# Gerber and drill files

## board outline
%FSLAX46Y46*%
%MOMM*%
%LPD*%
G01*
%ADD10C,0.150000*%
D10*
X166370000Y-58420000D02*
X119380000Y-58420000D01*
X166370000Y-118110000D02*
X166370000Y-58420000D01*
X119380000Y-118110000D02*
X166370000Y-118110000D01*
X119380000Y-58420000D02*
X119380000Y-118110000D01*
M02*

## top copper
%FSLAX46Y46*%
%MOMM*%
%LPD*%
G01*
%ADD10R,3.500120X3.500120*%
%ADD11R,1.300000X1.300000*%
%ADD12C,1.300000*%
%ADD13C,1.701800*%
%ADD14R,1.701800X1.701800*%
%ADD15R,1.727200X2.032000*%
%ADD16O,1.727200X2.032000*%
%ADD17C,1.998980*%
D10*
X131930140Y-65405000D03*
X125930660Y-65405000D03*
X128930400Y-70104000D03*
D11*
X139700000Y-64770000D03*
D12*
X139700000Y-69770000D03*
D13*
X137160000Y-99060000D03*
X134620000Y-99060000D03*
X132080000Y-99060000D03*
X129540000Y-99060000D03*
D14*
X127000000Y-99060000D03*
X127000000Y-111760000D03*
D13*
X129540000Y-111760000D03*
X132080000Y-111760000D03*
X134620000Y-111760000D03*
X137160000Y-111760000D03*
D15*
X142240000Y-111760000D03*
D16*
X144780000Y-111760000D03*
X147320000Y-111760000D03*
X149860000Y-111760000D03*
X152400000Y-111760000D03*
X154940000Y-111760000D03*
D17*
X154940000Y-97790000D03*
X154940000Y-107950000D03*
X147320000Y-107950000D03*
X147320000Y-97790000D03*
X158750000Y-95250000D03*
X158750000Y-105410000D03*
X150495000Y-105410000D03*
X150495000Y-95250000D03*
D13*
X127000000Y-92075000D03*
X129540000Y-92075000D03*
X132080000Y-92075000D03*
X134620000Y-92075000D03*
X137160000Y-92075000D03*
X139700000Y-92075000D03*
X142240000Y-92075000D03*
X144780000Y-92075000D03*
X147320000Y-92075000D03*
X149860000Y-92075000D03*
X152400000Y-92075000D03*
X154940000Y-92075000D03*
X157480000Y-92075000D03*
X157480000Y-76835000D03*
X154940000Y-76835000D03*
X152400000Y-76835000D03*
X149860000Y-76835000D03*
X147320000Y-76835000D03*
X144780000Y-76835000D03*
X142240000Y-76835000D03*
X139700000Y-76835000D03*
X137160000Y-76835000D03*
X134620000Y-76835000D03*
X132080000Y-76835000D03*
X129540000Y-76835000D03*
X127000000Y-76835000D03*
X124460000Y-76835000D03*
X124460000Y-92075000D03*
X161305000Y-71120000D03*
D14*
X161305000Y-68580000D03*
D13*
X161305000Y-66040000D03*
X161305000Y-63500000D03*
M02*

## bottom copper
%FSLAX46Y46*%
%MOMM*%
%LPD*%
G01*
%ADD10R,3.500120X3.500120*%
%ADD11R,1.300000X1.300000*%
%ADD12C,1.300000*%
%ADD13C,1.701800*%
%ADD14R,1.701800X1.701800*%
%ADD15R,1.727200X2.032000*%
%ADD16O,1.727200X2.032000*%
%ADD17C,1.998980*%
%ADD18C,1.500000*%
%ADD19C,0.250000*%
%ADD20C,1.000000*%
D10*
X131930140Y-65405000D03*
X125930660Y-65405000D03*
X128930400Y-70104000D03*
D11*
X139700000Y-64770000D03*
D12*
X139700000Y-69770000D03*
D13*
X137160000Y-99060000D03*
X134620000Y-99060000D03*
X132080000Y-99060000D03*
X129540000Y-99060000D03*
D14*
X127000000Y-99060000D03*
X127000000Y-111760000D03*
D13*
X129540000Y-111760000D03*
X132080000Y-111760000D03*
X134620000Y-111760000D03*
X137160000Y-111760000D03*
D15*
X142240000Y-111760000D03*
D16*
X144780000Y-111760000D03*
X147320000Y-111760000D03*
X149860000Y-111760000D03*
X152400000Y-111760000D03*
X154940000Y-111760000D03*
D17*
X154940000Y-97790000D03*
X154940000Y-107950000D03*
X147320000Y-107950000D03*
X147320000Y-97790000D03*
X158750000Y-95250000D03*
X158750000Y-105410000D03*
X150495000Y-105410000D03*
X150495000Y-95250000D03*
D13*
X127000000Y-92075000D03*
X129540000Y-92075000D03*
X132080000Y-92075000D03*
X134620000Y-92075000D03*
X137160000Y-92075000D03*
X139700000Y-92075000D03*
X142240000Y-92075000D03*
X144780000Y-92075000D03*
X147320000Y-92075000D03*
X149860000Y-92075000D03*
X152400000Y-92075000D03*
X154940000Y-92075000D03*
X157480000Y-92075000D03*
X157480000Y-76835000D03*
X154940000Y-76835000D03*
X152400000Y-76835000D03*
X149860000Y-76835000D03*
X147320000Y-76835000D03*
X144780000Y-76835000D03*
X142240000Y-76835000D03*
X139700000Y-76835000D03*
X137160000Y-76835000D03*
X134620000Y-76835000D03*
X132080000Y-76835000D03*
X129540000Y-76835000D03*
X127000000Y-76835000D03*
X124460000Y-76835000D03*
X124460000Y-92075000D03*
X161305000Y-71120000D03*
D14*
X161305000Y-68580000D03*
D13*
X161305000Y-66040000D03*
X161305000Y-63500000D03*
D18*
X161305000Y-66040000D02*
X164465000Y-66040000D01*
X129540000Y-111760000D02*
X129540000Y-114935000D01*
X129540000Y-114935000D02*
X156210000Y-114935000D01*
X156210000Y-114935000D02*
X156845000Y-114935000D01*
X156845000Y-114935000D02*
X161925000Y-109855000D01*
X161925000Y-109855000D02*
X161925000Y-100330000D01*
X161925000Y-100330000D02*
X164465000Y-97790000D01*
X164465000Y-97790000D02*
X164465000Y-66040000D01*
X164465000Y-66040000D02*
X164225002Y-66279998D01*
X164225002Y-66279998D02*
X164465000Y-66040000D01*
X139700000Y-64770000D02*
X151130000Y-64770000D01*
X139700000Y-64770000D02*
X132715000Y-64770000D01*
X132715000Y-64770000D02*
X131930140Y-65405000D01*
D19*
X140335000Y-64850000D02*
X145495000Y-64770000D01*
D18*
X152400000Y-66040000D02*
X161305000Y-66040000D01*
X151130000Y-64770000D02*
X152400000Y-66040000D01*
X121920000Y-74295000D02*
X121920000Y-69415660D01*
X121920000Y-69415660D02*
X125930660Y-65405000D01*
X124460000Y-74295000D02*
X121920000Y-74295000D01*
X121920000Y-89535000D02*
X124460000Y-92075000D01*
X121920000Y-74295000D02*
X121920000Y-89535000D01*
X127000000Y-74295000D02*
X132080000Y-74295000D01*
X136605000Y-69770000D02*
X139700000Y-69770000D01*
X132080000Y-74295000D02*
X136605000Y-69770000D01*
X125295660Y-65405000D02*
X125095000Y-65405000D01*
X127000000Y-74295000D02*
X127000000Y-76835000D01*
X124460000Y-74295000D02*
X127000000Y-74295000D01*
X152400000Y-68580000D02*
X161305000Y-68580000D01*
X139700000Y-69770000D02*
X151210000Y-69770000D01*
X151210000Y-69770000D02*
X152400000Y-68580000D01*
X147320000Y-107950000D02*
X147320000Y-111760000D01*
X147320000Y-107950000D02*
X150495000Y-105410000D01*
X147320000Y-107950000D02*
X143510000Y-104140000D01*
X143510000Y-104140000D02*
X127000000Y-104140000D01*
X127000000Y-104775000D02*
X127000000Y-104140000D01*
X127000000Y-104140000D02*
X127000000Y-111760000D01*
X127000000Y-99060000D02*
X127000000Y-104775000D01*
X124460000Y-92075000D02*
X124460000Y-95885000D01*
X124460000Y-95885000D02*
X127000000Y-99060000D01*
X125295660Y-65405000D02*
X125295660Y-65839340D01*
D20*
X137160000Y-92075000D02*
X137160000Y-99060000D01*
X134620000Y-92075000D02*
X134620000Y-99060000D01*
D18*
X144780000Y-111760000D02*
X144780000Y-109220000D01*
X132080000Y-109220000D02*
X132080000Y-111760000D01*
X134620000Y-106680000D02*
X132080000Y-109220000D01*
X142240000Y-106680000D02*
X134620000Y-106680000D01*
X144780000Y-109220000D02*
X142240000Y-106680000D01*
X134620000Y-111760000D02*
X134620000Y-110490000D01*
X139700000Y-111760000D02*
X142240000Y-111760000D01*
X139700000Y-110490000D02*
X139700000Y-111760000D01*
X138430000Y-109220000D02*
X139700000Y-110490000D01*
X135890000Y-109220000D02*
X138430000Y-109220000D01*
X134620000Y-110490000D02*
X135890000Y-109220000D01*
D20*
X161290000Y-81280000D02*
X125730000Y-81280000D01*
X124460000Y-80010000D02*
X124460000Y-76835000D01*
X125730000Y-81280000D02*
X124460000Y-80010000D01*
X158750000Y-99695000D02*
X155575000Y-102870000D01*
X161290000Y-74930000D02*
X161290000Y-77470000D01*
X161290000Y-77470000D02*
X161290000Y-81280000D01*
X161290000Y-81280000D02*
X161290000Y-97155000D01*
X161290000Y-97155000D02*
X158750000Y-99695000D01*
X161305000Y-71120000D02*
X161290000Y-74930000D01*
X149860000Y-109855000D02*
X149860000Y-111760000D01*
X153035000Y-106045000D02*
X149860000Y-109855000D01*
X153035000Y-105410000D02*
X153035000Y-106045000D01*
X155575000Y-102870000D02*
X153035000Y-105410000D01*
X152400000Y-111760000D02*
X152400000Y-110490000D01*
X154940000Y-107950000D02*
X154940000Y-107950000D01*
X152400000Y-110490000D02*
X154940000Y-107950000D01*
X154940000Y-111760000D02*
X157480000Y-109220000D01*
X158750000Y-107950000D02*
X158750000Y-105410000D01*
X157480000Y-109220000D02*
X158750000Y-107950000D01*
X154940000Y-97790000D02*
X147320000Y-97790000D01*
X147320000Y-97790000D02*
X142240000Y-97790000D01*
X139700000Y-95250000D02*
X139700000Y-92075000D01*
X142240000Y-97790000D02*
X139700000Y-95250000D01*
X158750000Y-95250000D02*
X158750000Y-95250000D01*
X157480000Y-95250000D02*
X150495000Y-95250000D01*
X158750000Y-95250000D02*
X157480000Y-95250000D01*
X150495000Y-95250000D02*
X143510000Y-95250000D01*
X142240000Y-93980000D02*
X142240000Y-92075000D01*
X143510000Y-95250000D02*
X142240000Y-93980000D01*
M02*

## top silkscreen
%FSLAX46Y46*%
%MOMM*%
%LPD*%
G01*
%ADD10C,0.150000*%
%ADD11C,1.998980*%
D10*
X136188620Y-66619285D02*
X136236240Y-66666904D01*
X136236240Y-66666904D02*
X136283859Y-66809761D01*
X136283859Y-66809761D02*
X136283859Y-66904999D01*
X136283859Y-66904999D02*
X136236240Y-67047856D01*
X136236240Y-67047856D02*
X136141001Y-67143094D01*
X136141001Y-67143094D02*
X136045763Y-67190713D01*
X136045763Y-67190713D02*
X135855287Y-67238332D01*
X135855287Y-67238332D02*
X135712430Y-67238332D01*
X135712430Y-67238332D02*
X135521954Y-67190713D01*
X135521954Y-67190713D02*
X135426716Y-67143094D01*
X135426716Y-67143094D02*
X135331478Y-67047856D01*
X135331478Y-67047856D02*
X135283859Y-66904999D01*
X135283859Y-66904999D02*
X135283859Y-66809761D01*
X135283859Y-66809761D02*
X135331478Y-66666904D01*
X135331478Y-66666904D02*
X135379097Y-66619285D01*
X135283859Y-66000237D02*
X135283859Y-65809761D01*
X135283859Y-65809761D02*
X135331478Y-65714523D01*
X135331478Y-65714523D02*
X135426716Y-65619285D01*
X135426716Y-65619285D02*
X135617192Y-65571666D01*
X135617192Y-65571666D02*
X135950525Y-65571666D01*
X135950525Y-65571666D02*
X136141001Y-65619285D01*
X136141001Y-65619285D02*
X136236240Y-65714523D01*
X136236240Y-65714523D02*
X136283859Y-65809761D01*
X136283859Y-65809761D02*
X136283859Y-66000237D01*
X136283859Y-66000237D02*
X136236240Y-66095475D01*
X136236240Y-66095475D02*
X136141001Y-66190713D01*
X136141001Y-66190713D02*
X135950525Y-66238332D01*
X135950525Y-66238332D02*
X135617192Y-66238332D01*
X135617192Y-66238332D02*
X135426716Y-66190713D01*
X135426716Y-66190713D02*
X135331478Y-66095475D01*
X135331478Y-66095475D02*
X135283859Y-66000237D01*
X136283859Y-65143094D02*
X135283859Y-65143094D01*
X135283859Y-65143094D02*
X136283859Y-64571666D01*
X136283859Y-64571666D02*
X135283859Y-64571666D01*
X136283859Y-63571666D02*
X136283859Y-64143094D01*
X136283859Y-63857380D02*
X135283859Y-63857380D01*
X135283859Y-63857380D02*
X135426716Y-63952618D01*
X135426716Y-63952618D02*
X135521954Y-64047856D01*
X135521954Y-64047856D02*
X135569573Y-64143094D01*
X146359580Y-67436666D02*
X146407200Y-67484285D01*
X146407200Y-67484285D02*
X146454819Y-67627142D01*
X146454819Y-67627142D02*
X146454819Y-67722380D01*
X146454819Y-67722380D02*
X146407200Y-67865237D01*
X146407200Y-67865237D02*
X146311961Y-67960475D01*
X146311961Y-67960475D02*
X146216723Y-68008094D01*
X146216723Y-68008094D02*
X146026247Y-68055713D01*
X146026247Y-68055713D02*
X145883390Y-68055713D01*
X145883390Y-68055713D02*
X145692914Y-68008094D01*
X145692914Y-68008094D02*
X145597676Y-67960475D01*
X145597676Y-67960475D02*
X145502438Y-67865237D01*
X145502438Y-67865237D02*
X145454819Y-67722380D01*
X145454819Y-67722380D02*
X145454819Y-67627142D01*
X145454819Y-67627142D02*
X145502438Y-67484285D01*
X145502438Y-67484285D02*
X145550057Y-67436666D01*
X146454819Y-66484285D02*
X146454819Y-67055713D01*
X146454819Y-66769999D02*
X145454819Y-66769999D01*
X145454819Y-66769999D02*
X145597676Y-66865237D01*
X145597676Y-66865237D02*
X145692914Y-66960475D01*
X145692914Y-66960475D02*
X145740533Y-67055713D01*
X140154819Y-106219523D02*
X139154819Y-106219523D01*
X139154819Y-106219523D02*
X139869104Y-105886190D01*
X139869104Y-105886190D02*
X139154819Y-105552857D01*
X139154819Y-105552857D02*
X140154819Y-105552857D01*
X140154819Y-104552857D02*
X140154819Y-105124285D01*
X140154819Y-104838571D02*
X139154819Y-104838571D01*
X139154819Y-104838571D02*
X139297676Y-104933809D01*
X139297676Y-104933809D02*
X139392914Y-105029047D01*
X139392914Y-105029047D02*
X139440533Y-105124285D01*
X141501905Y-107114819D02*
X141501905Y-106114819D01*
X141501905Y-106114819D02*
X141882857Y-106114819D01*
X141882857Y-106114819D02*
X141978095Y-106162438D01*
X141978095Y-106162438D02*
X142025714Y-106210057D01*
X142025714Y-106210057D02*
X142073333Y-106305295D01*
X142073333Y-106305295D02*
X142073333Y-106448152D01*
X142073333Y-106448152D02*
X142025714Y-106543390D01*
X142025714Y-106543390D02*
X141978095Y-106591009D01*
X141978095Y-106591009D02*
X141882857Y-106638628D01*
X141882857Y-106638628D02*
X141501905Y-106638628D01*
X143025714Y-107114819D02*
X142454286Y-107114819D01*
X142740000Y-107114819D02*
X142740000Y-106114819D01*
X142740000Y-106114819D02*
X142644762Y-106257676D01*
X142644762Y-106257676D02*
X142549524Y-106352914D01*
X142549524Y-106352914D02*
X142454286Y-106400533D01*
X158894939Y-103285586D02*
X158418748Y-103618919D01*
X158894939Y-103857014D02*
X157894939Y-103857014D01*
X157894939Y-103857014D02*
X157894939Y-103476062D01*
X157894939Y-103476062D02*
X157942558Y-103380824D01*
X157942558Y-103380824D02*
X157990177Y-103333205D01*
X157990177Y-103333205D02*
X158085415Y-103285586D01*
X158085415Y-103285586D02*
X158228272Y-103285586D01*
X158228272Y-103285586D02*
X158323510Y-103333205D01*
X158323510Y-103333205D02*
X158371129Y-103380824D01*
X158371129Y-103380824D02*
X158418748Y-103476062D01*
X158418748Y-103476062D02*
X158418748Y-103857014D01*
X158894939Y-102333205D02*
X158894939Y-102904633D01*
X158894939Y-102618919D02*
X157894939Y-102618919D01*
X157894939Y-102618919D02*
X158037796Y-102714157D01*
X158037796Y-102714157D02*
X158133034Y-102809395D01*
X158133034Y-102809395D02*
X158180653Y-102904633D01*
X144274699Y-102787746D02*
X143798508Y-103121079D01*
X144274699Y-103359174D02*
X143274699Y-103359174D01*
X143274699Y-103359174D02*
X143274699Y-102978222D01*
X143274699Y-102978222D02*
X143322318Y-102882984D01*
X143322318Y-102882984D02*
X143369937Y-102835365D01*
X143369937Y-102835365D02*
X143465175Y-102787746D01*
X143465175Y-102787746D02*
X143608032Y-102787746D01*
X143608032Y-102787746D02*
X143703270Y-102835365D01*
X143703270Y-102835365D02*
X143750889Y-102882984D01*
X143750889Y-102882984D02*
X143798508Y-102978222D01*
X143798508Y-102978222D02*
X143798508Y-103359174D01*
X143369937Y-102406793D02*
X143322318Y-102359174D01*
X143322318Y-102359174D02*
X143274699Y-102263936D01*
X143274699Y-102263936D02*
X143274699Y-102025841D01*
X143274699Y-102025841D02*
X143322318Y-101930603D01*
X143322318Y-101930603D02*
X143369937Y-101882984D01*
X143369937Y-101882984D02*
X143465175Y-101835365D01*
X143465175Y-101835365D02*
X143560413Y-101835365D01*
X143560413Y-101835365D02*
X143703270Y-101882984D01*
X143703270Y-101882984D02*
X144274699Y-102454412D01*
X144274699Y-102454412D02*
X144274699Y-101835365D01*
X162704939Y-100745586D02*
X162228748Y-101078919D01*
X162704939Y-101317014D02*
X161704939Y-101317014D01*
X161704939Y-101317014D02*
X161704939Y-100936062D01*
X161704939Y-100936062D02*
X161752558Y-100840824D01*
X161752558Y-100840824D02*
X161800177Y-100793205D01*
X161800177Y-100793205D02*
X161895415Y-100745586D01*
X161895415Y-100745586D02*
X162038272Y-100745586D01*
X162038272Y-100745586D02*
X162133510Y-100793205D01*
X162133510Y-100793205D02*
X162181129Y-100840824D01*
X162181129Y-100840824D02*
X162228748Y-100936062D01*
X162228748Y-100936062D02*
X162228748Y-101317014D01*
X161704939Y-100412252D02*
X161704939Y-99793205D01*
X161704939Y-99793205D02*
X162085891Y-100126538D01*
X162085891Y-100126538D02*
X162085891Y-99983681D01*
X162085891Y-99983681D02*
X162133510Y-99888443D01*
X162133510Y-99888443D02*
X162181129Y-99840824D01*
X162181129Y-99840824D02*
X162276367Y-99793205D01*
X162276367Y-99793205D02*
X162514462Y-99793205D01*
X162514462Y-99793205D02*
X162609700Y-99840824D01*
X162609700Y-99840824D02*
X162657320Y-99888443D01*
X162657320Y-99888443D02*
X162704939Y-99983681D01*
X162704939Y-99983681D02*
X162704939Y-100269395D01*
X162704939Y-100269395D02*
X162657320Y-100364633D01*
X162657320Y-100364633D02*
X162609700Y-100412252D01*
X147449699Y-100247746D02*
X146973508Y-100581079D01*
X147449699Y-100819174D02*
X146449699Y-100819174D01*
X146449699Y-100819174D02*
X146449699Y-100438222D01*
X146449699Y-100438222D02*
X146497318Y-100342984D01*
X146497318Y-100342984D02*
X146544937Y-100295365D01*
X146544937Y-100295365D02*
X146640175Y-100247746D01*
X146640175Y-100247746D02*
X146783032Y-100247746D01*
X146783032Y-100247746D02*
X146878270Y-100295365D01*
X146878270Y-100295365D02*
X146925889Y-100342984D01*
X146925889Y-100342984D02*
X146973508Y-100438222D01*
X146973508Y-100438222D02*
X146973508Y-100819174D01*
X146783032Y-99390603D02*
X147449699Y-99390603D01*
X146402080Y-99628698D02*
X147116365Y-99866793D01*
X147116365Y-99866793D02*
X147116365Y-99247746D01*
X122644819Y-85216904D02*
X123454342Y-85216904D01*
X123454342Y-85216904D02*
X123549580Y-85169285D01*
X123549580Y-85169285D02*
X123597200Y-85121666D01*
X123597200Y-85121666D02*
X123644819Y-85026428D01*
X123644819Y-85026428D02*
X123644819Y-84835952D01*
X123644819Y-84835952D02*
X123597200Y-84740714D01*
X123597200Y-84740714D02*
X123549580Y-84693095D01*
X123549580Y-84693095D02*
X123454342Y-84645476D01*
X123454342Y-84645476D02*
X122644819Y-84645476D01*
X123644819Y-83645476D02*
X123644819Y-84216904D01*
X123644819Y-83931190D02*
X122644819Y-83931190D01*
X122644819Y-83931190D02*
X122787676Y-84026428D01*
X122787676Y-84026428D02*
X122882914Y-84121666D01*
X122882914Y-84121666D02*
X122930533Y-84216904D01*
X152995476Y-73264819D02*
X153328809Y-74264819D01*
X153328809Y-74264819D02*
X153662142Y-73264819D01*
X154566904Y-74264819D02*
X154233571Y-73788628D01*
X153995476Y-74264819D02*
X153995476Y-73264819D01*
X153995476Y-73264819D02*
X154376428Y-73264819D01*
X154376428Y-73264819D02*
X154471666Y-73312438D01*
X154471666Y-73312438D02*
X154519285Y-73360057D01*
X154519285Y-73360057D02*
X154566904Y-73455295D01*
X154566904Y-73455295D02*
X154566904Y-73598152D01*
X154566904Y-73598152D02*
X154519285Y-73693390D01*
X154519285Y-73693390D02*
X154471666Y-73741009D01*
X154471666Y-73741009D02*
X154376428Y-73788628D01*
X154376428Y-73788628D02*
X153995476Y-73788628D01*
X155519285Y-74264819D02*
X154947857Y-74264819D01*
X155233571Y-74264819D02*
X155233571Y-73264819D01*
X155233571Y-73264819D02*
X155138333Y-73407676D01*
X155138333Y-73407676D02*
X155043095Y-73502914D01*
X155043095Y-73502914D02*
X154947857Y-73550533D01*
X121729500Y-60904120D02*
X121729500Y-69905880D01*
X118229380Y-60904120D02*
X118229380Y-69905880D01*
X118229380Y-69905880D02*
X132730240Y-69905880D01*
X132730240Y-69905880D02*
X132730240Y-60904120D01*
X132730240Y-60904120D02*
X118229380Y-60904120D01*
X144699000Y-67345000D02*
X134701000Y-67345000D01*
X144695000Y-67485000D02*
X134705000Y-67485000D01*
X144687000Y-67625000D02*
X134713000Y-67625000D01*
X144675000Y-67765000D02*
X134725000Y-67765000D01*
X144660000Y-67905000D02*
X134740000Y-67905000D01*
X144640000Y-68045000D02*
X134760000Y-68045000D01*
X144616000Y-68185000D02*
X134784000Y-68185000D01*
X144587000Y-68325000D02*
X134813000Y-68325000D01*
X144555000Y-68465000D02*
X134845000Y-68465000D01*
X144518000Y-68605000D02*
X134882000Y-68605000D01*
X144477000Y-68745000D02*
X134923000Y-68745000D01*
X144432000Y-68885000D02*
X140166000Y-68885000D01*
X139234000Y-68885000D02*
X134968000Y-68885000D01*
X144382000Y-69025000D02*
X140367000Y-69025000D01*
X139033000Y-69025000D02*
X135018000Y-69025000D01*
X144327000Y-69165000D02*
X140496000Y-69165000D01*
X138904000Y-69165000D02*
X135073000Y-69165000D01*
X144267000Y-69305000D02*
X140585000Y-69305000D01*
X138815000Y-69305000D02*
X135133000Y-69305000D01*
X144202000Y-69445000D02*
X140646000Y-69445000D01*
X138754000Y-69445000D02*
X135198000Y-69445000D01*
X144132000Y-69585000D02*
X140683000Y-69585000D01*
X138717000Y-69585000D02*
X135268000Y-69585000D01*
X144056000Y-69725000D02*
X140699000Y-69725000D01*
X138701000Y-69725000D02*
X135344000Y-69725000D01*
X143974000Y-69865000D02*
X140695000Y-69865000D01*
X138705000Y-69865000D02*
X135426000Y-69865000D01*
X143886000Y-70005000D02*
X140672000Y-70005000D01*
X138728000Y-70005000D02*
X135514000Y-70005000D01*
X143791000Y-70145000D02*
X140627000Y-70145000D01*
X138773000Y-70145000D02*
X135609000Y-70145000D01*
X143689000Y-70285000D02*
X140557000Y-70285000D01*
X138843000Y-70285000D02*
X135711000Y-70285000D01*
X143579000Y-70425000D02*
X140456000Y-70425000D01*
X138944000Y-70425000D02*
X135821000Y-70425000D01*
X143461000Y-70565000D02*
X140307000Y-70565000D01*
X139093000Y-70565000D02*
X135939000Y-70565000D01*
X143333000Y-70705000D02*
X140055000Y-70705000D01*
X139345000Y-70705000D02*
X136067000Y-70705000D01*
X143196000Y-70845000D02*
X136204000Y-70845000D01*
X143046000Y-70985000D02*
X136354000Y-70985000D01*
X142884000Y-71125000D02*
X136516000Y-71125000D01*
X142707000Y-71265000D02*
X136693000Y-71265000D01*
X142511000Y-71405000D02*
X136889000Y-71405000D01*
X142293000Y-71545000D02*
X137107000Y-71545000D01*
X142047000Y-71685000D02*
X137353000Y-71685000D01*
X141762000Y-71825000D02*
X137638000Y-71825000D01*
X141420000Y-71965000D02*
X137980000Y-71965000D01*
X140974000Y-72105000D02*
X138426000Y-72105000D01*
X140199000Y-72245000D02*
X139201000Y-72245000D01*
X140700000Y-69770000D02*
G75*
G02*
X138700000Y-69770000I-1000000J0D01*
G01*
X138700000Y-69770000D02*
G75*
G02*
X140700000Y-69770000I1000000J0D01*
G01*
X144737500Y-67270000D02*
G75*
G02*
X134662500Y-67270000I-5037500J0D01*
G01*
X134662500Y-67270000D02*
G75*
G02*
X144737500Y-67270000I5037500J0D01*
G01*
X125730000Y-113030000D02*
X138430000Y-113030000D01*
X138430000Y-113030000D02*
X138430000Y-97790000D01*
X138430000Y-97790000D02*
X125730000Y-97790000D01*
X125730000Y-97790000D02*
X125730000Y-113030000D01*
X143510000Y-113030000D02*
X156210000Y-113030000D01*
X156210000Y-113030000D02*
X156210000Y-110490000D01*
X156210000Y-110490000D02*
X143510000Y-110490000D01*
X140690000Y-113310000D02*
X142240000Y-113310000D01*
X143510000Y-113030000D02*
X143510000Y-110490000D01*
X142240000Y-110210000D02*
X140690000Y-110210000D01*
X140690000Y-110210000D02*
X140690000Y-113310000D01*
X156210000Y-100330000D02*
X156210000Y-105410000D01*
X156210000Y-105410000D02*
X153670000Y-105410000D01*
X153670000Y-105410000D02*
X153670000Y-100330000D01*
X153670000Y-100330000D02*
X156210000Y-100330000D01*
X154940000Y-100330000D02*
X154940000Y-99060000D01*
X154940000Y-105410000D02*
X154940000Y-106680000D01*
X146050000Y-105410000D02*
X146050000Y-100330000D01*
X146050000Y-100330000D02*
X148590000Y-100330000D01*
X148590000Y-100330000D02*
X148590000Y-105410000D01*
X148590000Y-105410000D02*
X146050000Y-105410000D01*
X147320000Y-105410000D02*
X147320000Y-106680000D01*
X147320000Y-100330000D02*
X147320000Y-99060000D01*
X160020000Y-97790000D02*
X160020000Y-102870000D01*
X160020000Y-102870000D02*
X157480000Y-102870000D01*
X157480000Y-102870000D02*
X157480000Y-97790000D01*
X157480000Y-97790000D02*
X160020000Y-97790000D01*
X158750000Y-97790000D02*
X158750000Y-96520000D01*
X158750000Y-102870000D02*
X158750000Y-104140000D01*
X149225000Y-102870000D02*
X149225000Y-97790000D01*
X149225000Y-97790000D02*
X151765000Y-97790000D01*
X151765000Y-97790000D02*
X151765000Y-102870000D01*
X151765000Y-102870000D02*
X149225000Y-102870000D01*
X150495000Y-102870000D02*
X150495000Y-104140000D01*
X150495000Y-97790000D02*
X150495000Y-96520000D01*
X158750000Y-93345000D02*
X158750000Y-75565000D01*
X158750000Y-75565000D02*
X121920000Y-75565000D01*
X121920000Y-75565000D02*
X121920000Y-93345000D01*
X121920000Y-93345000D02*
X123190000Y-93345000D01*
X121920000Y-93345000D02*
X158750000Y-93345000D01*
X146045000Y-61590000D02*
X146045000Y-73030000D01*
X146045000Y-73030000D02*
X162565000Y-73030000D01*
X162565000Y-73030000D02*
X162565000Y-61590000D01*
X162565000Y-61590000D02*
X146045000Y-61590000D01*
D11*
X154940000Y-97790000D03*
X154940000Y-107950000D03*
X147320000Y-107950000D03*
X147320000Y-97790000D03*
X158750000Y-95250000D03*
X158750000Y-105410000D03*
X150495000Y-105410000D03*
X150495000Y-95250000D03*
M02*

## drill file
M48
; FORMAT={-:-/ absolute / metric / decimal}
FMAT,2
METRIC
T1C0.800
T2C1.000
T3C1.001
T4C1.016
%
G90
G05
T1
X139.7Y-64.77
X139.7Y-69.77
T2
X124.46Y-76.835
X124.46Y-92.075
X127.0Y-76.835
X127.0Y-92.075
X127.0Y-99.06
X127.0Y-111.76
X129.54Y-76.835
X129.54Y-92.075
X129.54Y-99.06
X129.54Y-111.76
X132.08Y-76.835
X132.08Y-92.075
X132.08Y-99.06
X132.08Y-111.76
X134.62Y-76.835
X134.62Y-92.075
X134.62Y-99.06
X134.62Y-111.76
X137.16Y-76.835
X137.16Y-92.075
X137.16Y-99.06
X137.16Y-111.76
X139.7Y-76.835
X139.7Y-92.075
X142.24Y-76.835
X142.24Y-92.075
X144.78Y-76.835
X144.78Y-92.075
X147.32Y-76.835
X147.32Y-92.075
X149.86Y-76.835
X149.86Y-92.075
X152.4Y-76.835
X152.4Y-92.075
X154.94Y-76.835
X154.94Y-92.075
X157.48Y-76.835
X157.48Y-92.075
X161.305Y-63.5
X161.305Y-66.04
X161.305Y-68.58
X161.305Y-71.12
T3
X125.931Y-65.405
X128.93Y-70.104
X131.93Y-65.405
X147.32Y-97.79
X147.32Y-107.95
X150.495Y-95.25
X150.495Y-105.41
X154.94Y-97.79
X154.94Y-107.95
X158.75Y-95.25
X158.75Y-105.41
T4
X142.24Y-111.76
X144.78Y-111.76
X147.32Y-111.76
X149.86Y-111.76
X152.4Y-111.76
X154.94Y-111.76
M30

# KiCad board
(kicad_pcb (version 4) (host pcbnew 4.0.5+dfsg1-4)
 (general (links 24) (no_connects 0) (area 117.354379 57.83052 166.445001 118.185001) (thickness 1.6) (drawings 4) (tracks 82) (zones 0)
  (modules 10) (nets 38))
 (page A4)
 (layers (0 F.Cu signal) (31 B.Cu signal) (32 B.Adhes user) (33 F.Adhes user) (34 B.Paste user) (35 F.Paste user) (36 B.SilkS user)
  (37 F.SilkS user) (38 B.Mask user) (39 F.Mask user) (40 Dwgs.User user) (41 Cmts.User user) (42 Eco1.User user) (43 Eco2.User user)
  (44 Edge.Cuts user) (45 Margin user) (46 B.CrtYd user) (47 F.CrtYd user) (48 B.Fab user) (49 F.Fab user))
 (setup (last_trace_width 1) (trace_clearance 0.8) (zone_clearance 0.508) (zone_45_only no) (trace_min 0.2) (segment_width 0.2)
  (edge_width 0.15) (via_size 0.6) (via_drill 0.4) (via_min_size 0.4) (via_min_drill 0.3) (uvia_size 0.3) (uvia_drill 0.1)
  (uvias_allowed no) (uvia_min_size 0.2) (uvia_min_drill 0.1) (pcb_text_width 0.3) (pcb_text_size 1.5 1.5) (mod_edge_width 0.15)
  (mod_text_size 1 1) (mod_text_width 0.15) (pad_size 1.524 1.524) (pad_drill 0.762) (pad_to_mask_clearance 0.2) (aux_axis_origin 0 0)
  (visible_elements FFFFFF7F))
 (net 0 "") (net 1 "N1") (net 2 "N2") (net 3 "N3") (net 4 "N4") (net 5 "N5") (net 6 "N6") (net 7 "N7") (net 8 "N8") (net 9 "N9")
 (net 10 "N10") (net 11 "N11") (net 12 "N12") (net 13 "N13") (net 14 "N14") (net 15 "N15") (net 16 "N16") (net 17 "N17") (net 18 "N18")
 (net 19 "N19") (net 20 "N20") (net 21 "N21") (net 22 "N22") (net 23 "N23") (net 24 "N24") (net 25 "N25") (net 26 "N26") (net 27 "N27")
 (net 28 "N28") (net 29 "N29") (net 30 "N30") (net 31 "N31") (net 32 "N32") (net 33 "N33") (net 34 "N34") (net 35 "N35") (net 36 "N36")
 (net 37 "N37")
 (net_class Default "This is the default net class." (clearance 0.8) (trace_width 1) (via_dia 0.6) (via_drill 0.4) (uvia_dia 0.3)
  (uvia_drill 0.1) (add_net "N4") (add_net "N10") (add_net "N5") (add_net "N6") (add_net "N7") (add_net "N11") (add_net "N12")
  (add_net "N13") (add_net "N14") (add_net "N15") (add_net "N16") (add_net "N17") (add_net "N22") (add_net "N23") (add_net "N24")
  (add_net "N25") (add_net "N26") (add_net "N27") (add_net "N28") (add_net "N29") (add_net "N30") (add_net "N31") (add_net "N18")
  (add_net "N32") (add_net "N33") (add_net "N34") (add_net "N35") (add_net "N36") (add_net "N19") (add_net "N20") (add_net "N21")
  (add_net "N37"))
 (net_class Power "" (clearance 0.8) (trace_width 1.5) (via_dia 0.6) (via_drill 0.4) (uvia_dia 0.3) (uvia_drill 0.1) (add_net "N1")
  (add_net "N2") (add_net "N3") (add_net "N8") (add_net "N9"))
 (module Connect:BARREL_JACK (layer F.Cu) (at 125.73 65.405)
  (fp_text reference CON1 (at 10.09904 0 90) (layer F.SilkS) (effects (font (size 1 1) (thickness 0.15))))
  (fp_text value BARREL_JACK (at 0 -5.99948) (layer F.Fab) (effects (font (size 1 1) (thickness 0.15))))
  (fp_line (start -4.0005 -4.50088) (end -4.0005 4.50088) (layer F.SilkS) (width 0.15))
  (fp_line (start -7.50062 -4.50088) (end -7.50062 4.50088) (layer F.SilkS) (width 0.15))
  (fp_line (start -7.50062 4.50088) (end 7.00024 4.50088) (layer F.SilkS) (width 0.15))
  (fp_line (start 7.00024 4.50088) (end 7.00024 -4.50088) (layer F.SilkS) (width 0.15))
  (fp_line (start 7.00024 -4.50088) (end -7.50062 -4.50088) (layer F.SilkS) (width 0.15))
  (pad 1 thru_hole rect (at 6.20014 0) (size 3.50012 3.50012) (drill 1.00076) (layers *.Cu *.Mask) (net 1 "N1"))
  (pad 2 thru_hole rect (at 0.20066 0) (size 3.50012 3.50012) (drill 1.00076) (layers *.Cu *.Mask) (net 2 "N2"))
  (pad 3 thru_hole rect (at 3.2004 4.699) (size 3.50012 3.50012) (drill 1.00076) (layers *.Cu *.Mask) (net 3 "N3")))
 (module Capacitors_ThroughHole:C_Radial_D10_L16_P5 (layer F.Cu) (at 139.7 64.77 270)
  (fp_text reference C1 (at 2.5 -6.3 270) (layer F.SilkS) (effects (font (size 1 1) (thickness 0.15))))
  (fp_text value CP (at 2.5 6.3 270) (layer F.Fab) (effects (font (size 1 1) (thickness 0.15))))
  (fp_line (start 2.575 -4.999) (end 2.575 4.999) (layer F.SilkS) (width 0.15))
  (fp_line (start 2.715 -4.995) (end 2.715 4.995) (layer F.SilkS) (width 0.15))
  (fp_line (start 2.855 -4.987) (end 2.855 4.987) (layer F.SilkS) (width 0.15))
  (fp_line (start 2.995 -4.975) (end 2.995 4.975) (layer F.SilkS) (width 0.15))
  (fp_line (start 3.135 -4.96) (end 3.135 4.96) (layer F.SilkS) (width 0.15))
  (fp_line (start 3.275 -4.94) (end 3.275 4.94) (layer F.SilkS) (width 0.15))
  (fp_line (start 3.415 -4.916) (end 3.415 4.916) (layer F.SilkS) (width 0.15))
  (fp_line (start 3.555 -4.887) (end 3.555 4.887) (layer F.SilkS) (width 0.15))
  (fp_line (start 3.695 -4.855) (end 3.695 4.855) (layer F.SilkS) (width 0.15))
  (fp_line (start 3.835 -4.818) (end 3.835 4.818) (layer F.SilkS) (width 0.15))
  (fp_line (start 3.975 -4.777) (end 3.975 4.777) (layer F.SilkS) (width 0.15))
  (fp_line (start 4.115 -4.732) (end 4.115 -0.466) (layer F.SilkS) (width 0.15))
  (fp_line (start 4.115 0.466) (end 4.115 4.732) (layer F.SilkS) (width 0.15))
  (fp_line (start 4.255 -4.682) (end 4.255 -0.667) (layer F.SilkS) (width 0.15))
  (fp_line (start 4.255 0.667) (end 4.255 4.682) (layer F.SilkS) (width 0.15))
  (fp_line (start 4.395 -4.627) (end 4.395 -0.796) (layer F.SilkS) (width 0.15))
  (fp_line (start 4.395 0.796) (end 4.395 4.627) (layer F.SilkS) (width 0.15))
  (fp_line (start 4.535 -4.567) (end 4.535 -0.885) (layer F.SilkS) (width 0.15))
  (fp_line (start 4.535 0.885) (end 4.535 4.567) (layer F.SilkS) (width 0.15))
  (fp_line (start 4.675 -4.502) (end 4.675 -0.946) (layer F.SilkS) (width 0.15))
  (fp_line (start 4.675 0.946) (end 4.675 4.502) (layer F.SilkS) (width 0.15))
  (fp_line (start 4.815 -4.432) (end 4.815 -0.983) (layer F.SilkS) (width 0.15))
  (fp_line (start 4.815 0.983) (end 4.815 4.432) (layer F.SilkS) (width 0.15))
  (fp_line (start 4.955 -4.356) (end 4.955 -0.999) (layer F.SilkS) (width 0.15))
  (fp_line (start 4.955 0.999) (end 4.955 4.356) (layer F.SilkS) (width 0.15))
  (fp_line (start 5.095 -4.274) (end 5.095 -0.995) (layer F.SilkS) (width 0.15))
  (fp_line (start 5.095 0.995) (end 5.095 4.274) (layer F.SilkS) (width 0.15))
  (fp_line (start 5.235 -4.186) (end 5.235 -0.972) (layer F.SilkS) (width 0.15))
  (fp_line (start 5.235 0.972) (end 5.235 4.186) (layer F.SilkS) (width 0.15))
  (fp_line (start 5.375 -4.091) (end 5.375 -0.927) (layer F.SilkS) (width 0.15))
  (fp_line (start 5.375 0.927) (end 5.375 4.091) (layer F.SilkS) (width 0.15))
  (fp_line (start 5.515 -3.989) (end 5.515 -0.857) (layer F.SilkS) (width 0.15))
  (fp_line (start 5.515 0.857) (end 5.515 3.989) (layer F.SilkS) (width 0.15))
  (fp_line (start 5.655 -3.879) (end 5.655 -0.756) (layer F.SilkS) (width 0.15))
  (fp_line (start 5.655 0.756) (end 5.655 3.879) (layer F.SilkS) (width 0.15))
  (fp_line (start 5.795 -3.761) (end 5.795 -0.607) (layer F.SilkS) (width 0.15))
  (fp_line (start 5.795 0.607) (end 5.795 3.761) (layer F.SilkS) (width 0.15))
  (fp_line (start 5.935 -3.633) (end 5.935 -0.355) (layer F.SilkS) (width 0.15))
  (fp_line (start 5.935 0.355) (end 5.935 3.633) (layer F.SilkS) (width 0.15))
  (fp_line (start 6.075 -3.496) (end 6.075 3.496) (layer F.SilkS) (width 0.15))
  (fp_line (start 6.215 -3.346) (end 6.215 3.346) (layer F.SilkS) (width 0.15))
  (fp_line (start 6.355 -3.184) (end 6.355 3.184) (layer F.SilkS) (width 0.15))
  (fp_line (start 6.495 -3.007) (end 6.495 3.007) (layer F.SilkS) (width 0.15))
  (fp_line (start 6.635 -2.811) (end 6.635 2.811) (layer F.SilkS) (width 0.15))
  (fp_line (start 6.775 -2.593) (end 6.775 2.593) (layer F.SilkS) (width 0.15))
  (fp_line (start 6.915 -2.347) (end 6.915 2.347) (layer F.SilkS) (width 0.15))
  (fp_line (start 7.055 -2.062) (end 7.055 2.062) (layer F.SilkS) (width 0.15))
  (fp_line (start 7.195 -1.72) (end 7.195 1.72) (layer F.SilkS) (width 0.15))
  (fp_line (start 7.335 -1.274) (end 7.335 1.274) (layer F.SilkS) (width 0.15))
  (fp_line (start 7.475 -0.499) (end 7.475 0.499) (layer F.SilkS) (width 0.15))
  (fp_circle (center 5 0) (end 5 -1) (layer F.SilkS) (width 0.15))
  (fp_circle (center 2.5 0) (end 2.5 -5.0375) (layer F.SilkS) (width 0.15))
  (pad 1 thru_hole rect (at 0 0 270) (size 1.3 1.3) (drill 0.8) (layers *.Cu *.Mask) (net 1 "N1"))
  (pad 2 thru_hole circle (at 5 0 270) (size 1.3 1.3) (drill 0.8) (layers *.Cu *.Mask) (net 2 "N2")))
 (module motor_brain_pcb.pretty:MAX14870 (layer F.Cu) (at 132.08 105.41 270)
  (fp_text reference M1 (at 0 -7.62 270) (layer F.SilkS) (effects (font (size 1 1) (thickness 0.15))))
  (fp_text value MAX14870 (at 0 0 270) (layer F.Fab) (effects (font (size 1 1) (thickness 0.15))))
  (fp_line (start 7.62 6.35) (end 7.62 -6.35) (layer F.SilkS) (width 0.15))
  (fp_line (start 7.62 -6.35) (end -7.62 -6.35) (layer F.SilkS) (width 0.15))
  (fp_line (start -7.62 -6.35) (end -7.62 6.35) (layer F.SilkS) (width 0.15))
  (fp_line (start -7.62 6.35) (end 7.62 6.35) (layer F.SilkS) (width 0.15))
  (pad 1 thru_hole circle (at -6.35 -5.08 270) (size 1.7018 1.7018) (drill 1) (layers *.Cu *.Mask) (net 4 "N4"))
  (pad 2 thru_hole circle (at -6.35 -2.54 270) (size 1.7018 1.7018) (drill 1) (layers *.Cu *.Mask) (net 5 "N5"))
  (pad 3 thru_hole circle (at -6.35 0 270) (size 1.7018 1.7018) (drill 1) (layers *.Cu *.Mask) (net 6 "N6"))
  (pad 4 thru_hole circle (at -6.35 2.54 270) (size 1.7018 1.7018) (drill 1) (layers *.Cu *.Mask) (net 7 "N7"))
  (pad 5 thru_hole rect (at -6.35 5.08 270) (size 1.7018 1.7018) (drill 1) (layers *.Cu *.Mask) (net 2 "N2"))
  (pad 6 thru_hole rect (at 6.35 5.08 270) (size 1.7018 1.7018) (drill 1) (layers *.Cu *.Mask) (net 2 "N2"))
  (pad 7 thru_hole circle (at 6.35 2.54 270) (size 1.7018 1.7018) (drill 1) (layers *.Cu *.Mask) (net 1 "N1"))
  (pad 8 thru_hole circle (at 6.35 0 270) (size 1.7018 1.70184) (drill 1) (layers *.Cu *.Mask) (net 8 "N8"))
  (pad 9 thru_hole circle (at 6.35 -2.54 270) (size 1.7018 1.7018) (drill 1) (layers *.Cu *.Mask) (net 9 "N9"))
  (pad 10 thru_hole circle (at 6.35 -5.08 270) (size 1.7018 1.7018) (drill 1) (layers *.Cu *.Mask) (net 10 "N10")))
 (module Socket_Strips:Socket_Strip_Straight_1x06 (layer F.Cu) (at 142.24 111.76)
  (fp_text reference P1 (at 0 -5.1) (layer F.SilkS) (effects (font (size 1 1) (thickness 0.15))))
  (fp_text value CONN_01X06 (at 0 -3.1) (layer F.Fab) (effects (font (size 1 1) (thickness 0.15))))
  (fp_line (start 1.27 1.27) (end 13.97 1.27) (layer F.SilkS) (width 0.15))
  (fp_line (start 13.97 1.27) (end 13.97 -1.27) (layer F.SilkS) (width 0.15))
  (fp_line (start 13.97 -1.27) (end 1.27 -1.27) (layer F.SilkS) (width 0.15))
  (fp_line (start -1.55 1.55) (end 0 1.55) (layer F.SilkS) (width 0.15))
  (fp_line (start 1.27 1.27) (end 1.27 -1.27) (layer F.SilkS) (width 0.15))
  (fp_line (start 0 -1.55) (end -1.55 -1.55) (layer F.SilkS) (width 0.15))
  (fp_line (start -1.55 -1.55) (end -1.55 1.55) (layer F.SilkS) (width 0.15))
  (pad 1 thru_hole rect (at 0 0) (size 1.7272 2.032) (drill 1.016) (layers *.Cu *.Mask) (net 9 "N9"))
  (pad 2 thru_hole oval (at 2.54 0) (size 1.7272 2.032) (drill 1.016) (layers *.Cu *.Mask) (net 8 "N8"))
  (pad 3 thru_hole oval (at 5.08 0) (size 1.7272 2.032) (drill 1.016) (layers *.Cu *.Mask) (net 2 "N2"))
  (pad 4 thru_hole oval (at 7.62 0) (size 1.7272 2.032) (drill 1.016) (layers *.Cu *.Mask) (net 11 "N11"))
  (pad 5 thru_hole oval (at 10.16 0) (size 1.7272 2.032) (drill 1.016) (layers *.Cu *.Mask) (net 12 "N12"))
  (pad 6 thru_hole oval (at 12.7 0) (size 1.7272 2.032) (drill 1.016) (layers *.Cu *.Mask) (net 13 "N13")))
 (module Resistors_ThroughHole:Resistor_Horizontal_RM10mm (layer F.Cu) (at 154.94 97.79 270)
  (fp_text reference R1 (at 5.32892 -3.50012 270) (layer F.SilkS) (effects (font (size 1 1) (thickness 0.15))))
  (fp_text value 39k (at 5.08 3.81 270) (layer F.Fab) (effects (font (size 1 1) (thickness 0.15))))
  (fp_line (start 2.54 -1.27) (end 7.62 -1.27) (layer F.SilkS) (width 0.15))
  (fp_line (start 7.62 -1.27) (end 7.62 1.27) (layer F.SilkS) (width 0.15))
  (fp_line (start 7.62 1.27) (end 2.54 1.27) (layer F.SilkS) (width 0.15))
  (fp_line (start 2.54 1.27) (end 2.54 -1.27) (layer F.SilkS) (width 0.15))
  (fp_line (start 2.54 0) (end 1.27 0) (layer F.SilkS) (width 0.15))
  (fp_line (start 7.62 0) (end 8.89 0) (layer F.SilkS) (width 0.15))
  (pad 1 thru_hole circle (at 0 0 270) (size 1.99898 1.99898) (drill 1.00076) (layers *.Cu *.SilkS *.Mask) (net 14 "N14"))
  (pad 2 thru_hole circle (at 10.16 0 270) (size 1.99898 1.99898) (drill 1.00076) (layers *.Cu *.SilkS *.Mask) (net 12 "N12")))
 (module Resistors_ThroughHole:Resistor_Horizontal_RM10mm (layer F.Cu) (at 147.32 107.95 90)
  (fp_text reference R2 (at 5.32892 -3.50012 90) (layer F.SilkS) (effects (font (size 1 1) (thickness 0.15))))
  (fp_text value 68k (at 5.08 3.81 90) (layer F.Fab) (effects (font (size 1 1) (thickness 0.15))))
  (fp_line (start 2.54 -1.27) (end 7.62 -1.27) (layer F.SilkS) (width 0.15))
  (fp_line (start 7.62 -1.27) (end 7.62 1.27) (layer F.SilkS) (width 0.15))
  (fp_line (start 7.62 1.27) (end 2.54 1.27) (layer F.SilkS) (width 0.15))
  (fp_line (start 2.54 1.27) (end 2.54 -1.27) (layer F.SilkS) (width 0.15))
  (fp_line (start 2.54 0) (end 1.27 0) (layer F.SilkS) (width 0.15))
  (fp_line (start 7.62 0) (end 8.89 0) (layer F.SilkS) (width 0.15))
  (pad 1 thru_hole circle (at 0 0 90) (size 1.99898 1.99898) (drill 1.00076) (layers *.Cu *.SilkS *.Mask) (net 2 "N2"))
  (pad 2 thru_hole circle (at 10.16 0 90) (size 1.99898 1.99898) (drill 1.00076) (layers *.Cu *.SilkS *.Mask) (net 14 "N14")))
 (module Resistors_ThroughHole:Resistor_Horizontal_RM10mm (layer F.Cu) (at 158.75 95.25 270)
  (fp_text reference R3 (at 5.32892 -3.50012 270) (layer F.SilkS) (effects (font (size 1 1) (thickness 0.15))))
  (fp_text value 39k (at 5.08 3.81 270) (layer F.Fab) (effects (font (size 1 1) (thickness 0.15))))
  (fp_line (start 2.54 -1.27) (end 7.62 -1.27) (layer F.SilkS) (width 0.15))
  (fp_line (start 7.62 -1.27) (end 7.62 1.27) (layer F.SilkS) (width 0.15))
  (fp_line (start 7.62 1.27) (end 2.54 1.27) (layer F.SilkS) (width 0.15))
  (fp_line (start 2.54 1.27) (end 2.54 -1.27) (layer F.SilkS) (width 0.15))
  (fp_line (start 2.54 0) (end 1.27 0) (layer F.SilkS) (width 0.15))
  (fp_line (start 7.62 0) (end 8.89 0) (layer F.SilkS) (width 0.15))
  (pad 1 thru_hole circle (at 0 0 270) (size 1.99898 1.99898) (drill 1.00076) (layers *.Cu *.SilkS *.Mask) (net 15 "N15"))
  (pad 2 thru_hole circle (at 10.16 0 270) (size 1.99898 1.99898) (drill 1.00076) (layers *.Cu *.SilkS *.Mask) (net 13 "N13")))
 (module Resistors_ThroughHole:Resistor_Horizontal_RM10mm (layer F.Cu) (at 150.495 105.41 90)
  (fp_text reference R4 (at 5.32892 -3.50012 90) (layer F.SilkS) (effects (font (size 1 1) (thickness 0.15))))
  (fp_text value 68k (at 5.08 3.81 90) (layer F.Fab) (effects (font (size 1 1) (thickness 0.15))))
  (fp_line (start 2.54 -1.27) (end 7.62 -1.27) (layer F.SilkS) (width 0.15))
  (fp_line (start 7.62 -1.27) (end 7.62 1.27) (layer F.SilkS) (width 0.15))
  (fp_line (start 7.62 1.27) (end 2.54 1.27) (layer F.SilkS) (width 0.15))
  (fp_line (start 2.54 1.27) (end 2.54 -1.27) (layer F.SilkS) (width 0.15))
  (fp_line (start 2.54 0) (end 1.27 0) (layer F.SilkS) (width 0.15))
  (fp_line (start 7.62 0) (end 8.89 0) (layer F.SilkS) (width 0.15))
  (pad 1 thru_hole circle (at 0 0 90) (size 1.99898 1.99898) (drill 1.00076) (layers *.Cu *.SilkS *.Mask) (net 2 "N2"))
  (pad 2 thru_hole circle (at 10.16 0 90) (size 1.99898 1.99898) (drill 1.00076) (layers *.Cu *.SilkS *.Mask) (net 15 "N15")))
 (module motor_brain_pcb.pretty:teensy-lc (layer F.Cu) (at 139.7 84.455 90)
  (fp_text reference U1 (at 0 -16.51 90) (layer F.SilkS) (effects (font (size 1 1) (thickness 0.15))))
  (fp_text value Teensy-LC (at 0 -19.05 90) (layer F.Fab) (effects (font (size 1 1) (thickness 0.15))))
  (fp_line (start -8.89 19.05) (end 8.89 19.05) (layer F.SilkS) (width 0.15))
  (fp_line (start 8.89 19.05) (end 8.89 -17.78) (layer F.SilkS) (width 0.15))
  (fp_line (start 8.89 -17.78) (end -8.89 -17.78) (layer F.SilkS) (width 0.15))
  (fp_line (start -8.89 -17.78) (end -8.89 -16.51) (layer F.SilkS) (width 0.15))
  (fp_line (start -8.89 -17.78) (end -8.89 19.05) (layer F.SilkS) (width 0.15))
  (pad 0 thru_hole circle (at -7.62 -12.7 90) (size 1.7018 1.7018) (drill 1) (layers *.Cu *.Mask) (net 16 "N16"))
  (pad 1 thru_hole circle (at -7.62 -10.16 90) (size 1.7018 1.7018) (drill 1) (layers *.Cu *.Mask) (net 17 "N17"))
  (pad 2 thru_hole circle (at -7.62 -7.62 90) (size 1.7018 1.7018) (drill 1) (layers *.Cu *.Mask) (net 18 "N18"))
  (pad 3 thru_hole circle (at -7.62 -5.08 90) (size 1.7018 1.7018) (drill 1) (layers *.Cu *.Mask) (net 5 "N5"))
  (pad 4 thru_hole circle (at -7.62 -2.54 90) (size 1.7018 1.7018) (drill 1) (layers *.Cu *.Mask) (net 4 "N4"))
  (pad 5 thru_hole circle (at -7.62 0 90) (size 1.7018 1.7018) (drill 1) (layers *.Cu *.Mask) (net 14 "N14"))
  (pad 6 thru_hole circle (at -7.62 2.54 90) (size 1.7018 1.7018) (drill 1) (layers *.Cu *.Mask) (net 15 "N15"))
  (pad 7 thru_hole circle (at -7.62 5.08 90) (size 1.7018 1.7018) (drill 1) (layers *.Cu *.Mask) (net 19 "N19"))
  (pad 8 thru_hole circle (at -7.62 7.62 90) (size 1.7018 1.7018) (drill 1) (layers *.Cu *.Mask) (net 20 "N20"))
  (pad 9 thru_hole circle (at -7.62 10.16 90) (size 1.7018 1.7018) (drill 1) (layers *.Cu *.Mask) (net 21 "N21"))
  (pad 10 thru_hole circle (at -7.62 12.7 90) (size 1.7018 1.7018) (drill 1) (layers *.Cu *.Mask) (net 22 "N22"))
  (pad 11 thru_hole circle (at -7.62 15.24 90) (size 1.7018 1.7018) (drill 1) (layers *.Cu *.Mask) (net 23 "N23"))
  (pad 12 thru_hole circle (at -7.62 17.78 90) (size 1.7018 1.7018) (drill 1) (layers *.Cu *.Mask) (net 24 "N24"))
  (pad 13 thru_hole circle (at 7.62 17.78 90) (size 1.7018 1.7018) (drill 1) (layers *.Cu *.Mask) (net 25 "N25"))
  (pad 14 thru_hole circle (at 7.62 15.24 90) (size 1.7018 1.7018) (drill 1) (layers *.Cu *.Mask) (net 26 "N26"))
  (pad 15 thru_hole circle (at 7.62 12.7 90) (size 1.7018 1.7018) (drill 1) (layers *.Cu *.Mask) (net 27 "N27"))
  (pad 16 thru_hole circle (at 7.62 10.16 90) (size 1.7018 1.7018) (drill 1) (layers *.Cu *.Mask) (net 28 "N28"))
  (pad 17 thru_hole circle (at 7.62 7.62 90) (size 1.7018 1.7018) (drill 1) (layers *.Cu *.Mask) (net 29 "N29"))
  (pad 18 thru_hole circle (at 7.62 5.08 90) (size 1.7018 1.7018) (drill 1) (layers *.Cu *.Mask) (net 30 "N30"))
  (pad 19 thru_hole circle (at 7.62 2.54 90) (size 1.7018 1.7018) (drill 1) (layers *.Cu *.Mask) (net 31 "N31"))
  (pad 20 thru_hole circle (at 7.62 0 90) (size 1.7018 1.7018) (drill 1) (layers *.Cu *.Mask) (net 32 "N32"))
  (pad 21 thru_hole circle (at 7.62 -2.54 90) (size 1.7018 1.7018) (drill 1) (layers *.Cu *.Mask) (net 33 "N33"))
  (pad 22 thru_hole circle (at 7.62 -5.08 90) (size 1.7018 1.7018) (drill 1) (layers *.Cu *.Mask) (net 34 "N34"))
  (pad 23 thru_hole circle (at 7.62 -7.62 90) (size 1.7018 1.7018) (drill 1) (layers *.Cu *.Mask) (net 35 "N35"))
  (pad 24 thru_hole circle (at 7.62 -10.16 90) (size 1.7018 1.7018) (drill 1) (layers *.Cu *.Mask) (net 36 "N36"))
  (pad 25 thru_hole circle (at 7.62 -12.7 90) (size 1.7018 1.7018) (drill 1) (layers *.Cu *.Mask) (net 2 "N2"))
  (pad 26 thru_hole circle (at 7.62 -15.24 90) (size 1.7018 1.7018) (drill 1) (layers *.Cu *.Mask) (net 11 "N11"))
  (pad 27 thru_hole circle (at -7.62 -15.24 90) (size 1.7018 1.7018) (drill 1) (layers *.Cu *.Mask) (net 2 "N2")))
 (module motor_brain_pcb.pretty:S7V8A (layer F.Cu) (at 154.305 67.31 180)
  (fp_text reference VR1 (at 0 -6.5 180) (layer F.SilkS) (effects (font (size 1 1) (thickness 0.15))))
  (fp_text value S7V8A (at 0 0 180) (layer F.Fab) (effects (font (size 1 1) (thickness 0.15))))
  (fp_line (start 8.26 5.72) (end 8.26 -5.72) (layer F.SilkS) (width 0.15))
  (fp_line (start 8.26 -5.72) (end -8.26 -5.72) (layer F.SilkS) (width 0.15))
  (fp_line (start -8.26 -5.72) (end -8.26 5.72) (layer F.SilkS) (width 0.15))
  (fp_line (start -8.26 5.72) (end 8.26 5.72) (layer F.SilkS) (width 0.15))
  (pad 1 thru_hole circle (at -7 -3.81 180) (size 1.7018 1.7018) (drill 1) (layers *.Cu *.Mask) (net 11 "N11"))
  (pad 2 thru_hole rect (at -7 -1.27 180) (size 1.7018 1.7018) (drill 1) (layers *.Cu *.Mask) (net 2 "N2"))
  (pad 3 thru_hole circle (at -7 1.27 180) (size 1.7018 1.7018) (drill 1) (layers *.Cu *.Mask) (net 1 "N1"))
  (pad 4 thru_hole circle (at -7 3.81 180) (size 1.7018 1.7018) (drill 1) (layers *.Cu *.Mask) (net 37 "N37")))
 (gr_line (start 166.37 58.42) (end 119.38 58.42) (angle 90) (layer Edge.Cuts) (width 0.15))
 (gr_line (start 166.37 118.11) (end 166.37 58.42) (angle 90) (layer Edge.Cuts) (width 0.15))
 (gr_line (start 119.38 118.11) (end 166.37 118.11) (angle 90) (layer Edge.Cuts) (width 0.15))
 (gr_line (start 119.38 58.42) (end 119.38 118.11) (angle 90) (layer Edge.Cuts) (width 0.15))
 (segment (start 161.305 66.04) (end 164.465 66.04) (width 1.5) (layer B.Cu) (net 1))
 (segment (start 129.54 111.76) (end 129.54 114.935) (width 1.5) (layer B.Cu) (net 1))
 (segment (start 129.54 114.935) (end 156.21 114.935) (width 1.5) (layer B.Cu) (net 1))
 (segment (start 156.21 114.935) (end 156.845 114.935) (width 1.5) (layer B.Cu) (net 1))
 (segment (start 156.845 114.935) (end 161.925 109.855) (width 1.5) (layer B.Cu) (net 1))
 (segment (start 161.925 109.855) (end 161.925 100.33) (width 1.5) (layer B.Cu) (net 1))
 (segment (start 161.925 100.33) (end 164.465 97.79) (width 1.5) (layer B.Cu) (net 1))
 (segment (start 164.465 97.79) (end 164.465 66.04) (width 1.5) (layer B.Cu) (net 1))
 (segment (start 164.465 66.04) (end 164.225002 66.279998) (width 1.5) (layer B.Cu) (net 1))
 (segment (start 164.225002 66.279998) (end 164.465 66.04) (width 1.5) (layer B.Cu) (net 1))
 (segment (start 139.7 64.77) (end 151.13 64.77) (width 1.5) (layer B.Cu) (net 1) (status 10))
 (segment (start 139.7 64.77) (end 132.715 64.77) (width 1.5) (layer B.Cu) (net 1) (status 20))
 (segment (start 132.715 64.77) (end 131.93014 65.405) (width 1.5) (layer B.Cu) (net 1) (status 30))
 (segment (start 140.335 64.85) (end 145.495 64.77) (width 0.25) (layer B.Cu) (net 1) (status 10))
 (segment (start 152.4 66.04) (end 161.305 66.04) (width 1.5) (layer B.Cu) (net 1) (status 20))
 (segment (start 151.13 64.77) (end 152.4 66.04) (width 1.5) (layer B.Cu) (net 1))
 (segment (start 121.92 74.295) (end 121.92 69.41566) (width 1.5) (layer B.Cu) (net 2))
 (segment (start 121.92 69.41566) (end 125.93066 65.405) (width 1.5) (layer B.Cu) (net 2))
 (segment (start 124.46 74.295) (end 121.92 74.295) (width 1.5) (layer B.Cu) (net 2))
 (segment (start 121.92 89.535) (end 124.46 92.075) (width 1.5) (layer B.Cu) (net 2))
 (segment (start 121.92 74.295) (end 121.92 89.535) (width 1.5) (layer B.Cu) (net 2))
 (segment (start 127 74.295) (end 132.08 74.295) (width 1.5) (layer B.Cu) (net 2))
 (segment (start 136.605 69.77) (end 139.7 69.77) (width 1.5) (layer B.Cu) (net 2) (status 20))
 (segment (start 132.08 74.295) (end 136.605 69.77) (width 1.5) (layer B.Cu) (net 2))
 (segment (start 125.29566 65.405) (end 125.095 65.405) (width 1.5) (layer B.Cu) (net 2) (status 30))
 (segment (start 127 74.295) (end 127 76.835) (width 1.5) (layer B.Cu) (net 2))
 (segment (start 124.46 74.295) (end 127 74.295) (width 1.5) (layer B.Cu) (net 2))
 (segment (start 152.4 68.58) (end 161.305 68.58) (width 1.5) (layer B.Cu) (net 2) (status 20))
 (segment (start 139.7 69.77) (end 151.21 69.77) (width 1.5) (layer B.Cu) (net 2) (status 10))
 (segment (start 151.21 69.77) (end 152.4 68.58) (width 1.5) (layer B.Cu) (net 2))
 (segment (start 147.32 107.95) (end 147.32 111.76) (width 1.5) (layer B.Cu) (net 2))
 (segment (start 147.32 107.95) (end 150.495 105.41) (width 1.5) (layer B.Cu) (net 2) (status 20))
 (segment (start 147.32 107.95) (end 143.51 104.14) (width 1.5) (layer B.Cu) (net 2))
 (segment (start 143.51 104.14) (end 127 104.14) (width 1.5) (layer B.Cu) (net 2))
 (segment (start 127 104.775) (end 127 104.14) (width 1.5) (layer B.Cu) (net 2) (status 20))
 (segment (start 127 104.14) (end 127 111.76) (width 1.5) (layer B.Cu) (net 2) (status 20))
 (segment (start 127 99.06) (end 127 104.775) (width 1.5) (layer B.Cu) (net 2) (status 10))
 (segment (start 124.46 92.075) (end 124.46 95.885) (width 1.5) (layer B.Cu) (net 2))
 (segment (start 124.46 95.885) (end 127 99.06) (width 1.5) (layer B.Cu) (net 2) (status 20))
 (segment (start 125.29566 65.405) (end 125.29566 65.83934) (width 1.5) (layer B.Cu) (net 2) (status 30))
 (segment (start 137.16 92.075) (end 137.16 99.06) (width 1) (layer B.Cu) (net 4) (status 20))
 (segment (start 134.62 92.075) (end 134.62 99.06) (width 1) (layer B.Cu) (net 5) (status 20))
 (segment (start 144.78 111.76) (end 144.78 109.22) (width 1.5) (layer B.Cu) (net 8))
 (segment (start 132.08 109.22) (end 132.08 111.76) (width 1.5) (layer B.Cu) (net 8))
 (segment (start 134.62 106.68) (end 132.08 109.22) (width 1.5) (layer B.Cu) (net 8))
 (segment (start 142.24 106.68) (end 134.62 106.68) (width 1.5) (layer B.Cu) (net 8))
 (segment (start 144.78 109.22) (end 142.24 106.68) (width 1.5) (layer B.Cu) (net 8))
 (segment (start 134.62 111.76) (end 134.62 110.49) (width 1.5) (layer B.Cu) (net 9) (status 10))
 (segment (start 139.7 111.76) (end 142.24 111.76) (width 1.5) (layer B.Cu) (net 9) (status 20))
 (segment (start 139.7 110.49) (end 139.7 111.76) (width 1.5) (layer B.Cu) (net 9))
 (segment (start 138.43 109.22) (end 139.7 110.49) (width 1.5) (layer B.Cu) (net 9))
 (segment (start 135.89 109.22) (end 138.43 109.22) (width 1.5) (layer B.Cu) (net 9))
 (segment (start 134.62 110.49) (end 135.89 109.22) (width 1.5) (layer B.Cu) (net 9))
 (segment (start 161.29 81.28) (end 125.73 81.28) (width 1) (layer B.Cu) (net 11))
 (segment (start 124.46 80.01) (end 124.46 76.835) (width 1) (layer B.Cu) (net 11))
 (segment (start 125.73 81.28) (end 124.46 80.01) (width 1) (layer B.Cu) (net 11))
 (segment (start 158.75 99.695) (end 155.575 102.87) (width 1) (layer B.Cu) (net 11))
 (segment (start 161.29 74.93) (end 161.29 77.47) (width 1) (layer B.Cu) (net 11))
 (segment (start 161.29 77.47) (end 161.29 81.28) (width 1) (layer B.Cu) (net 11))
 (segment (start 161.29 81.28) (end 161.29 97.155) (width 1) (layer B.Cu) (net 11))
 (segment (start 161.29 97.155) (end 158.75 99.695) (width 1) (layer B.Cu) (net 11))
 (segment (start 161.305 71.12) (end 161.29 74.93) (width 1) (layer B.Cu) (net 11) (status 10))
 (segment (start 149.86 109.855) (end 149.86 111.76) (width 1) (layer B.Cu) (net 11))
 (segment (start 153.035 106.045) (end 149.86 109.855) (width 1) (layer B.Cu) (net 11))
 (segment (start 153.035 105.41) (end 153.035 106.045) (width 1) (layer B.Cu) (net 11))
 (segment (start 155.575 102.87) (end 153.035 105.41) (width 1) (layer B.Cu) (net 11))
 (segment (start 152.4 111.76) (end 152.4 110.49) (width 1) (layer B.Cu) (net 12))
 (segment (start 154.94 107.95) (end 154.94 107.95) (width 1) (layer B.Cu) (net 12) (status 20))
 (segment (start 152.4 110.49) (end 154.94 107.95) (width 1) (layer B.Cu) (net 12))
 (segment (start 154.94 111.76) (end 157.48 109.22) (width 1) (layer B.Cu) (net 13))
 (segment (start 158.75 107.95) (end 158.75 105.41) (width 1) (layer B.Cu) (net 13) (status 20))
 (segment (start 157.48 109.22) (end 158.75 107.95) (width 1) (layer B.Cu) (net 13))
 (segment (start 154.94 97.79) (end 147.32 97.79) (width 1) (layer B.Cu) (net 14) (status 10))
 (segment (start 147.32 97.79) (end 142.24 97.79) (width 1) (layer B.Cu) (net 14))
 (segment (start 139.7 95.25) (end 139.7 92.075) (width 1) (layer B.Cu) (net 14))
 (segment (start 142.24 97.79) (end 139.7 95.25) (width 1) (layer B.Cu) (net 14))
 (segment (start 158.75 95.25) (end 158.75 95.25) (width 1) (layer B.Cu) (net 15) (status 10))
 (segment (start 157.48 95.25) (end 150.495 95.25) (width 1) (layer B.Cu) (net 15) (status 20))
 (segment (start 158.75 95.25) (end 157.48 95.25) (width 1) (layer B.Cu) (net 15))
 (segment (start 150.495 95.25) (end 143.51 95.25) (width 1) (layer B.Cu) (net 15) (status 10))
 (segment (start 142.24 93.98) (end 142.24 92.075) (width 1) (layer B.Cu) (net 15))
 (segment (start 143.51 95.25) (end 142.24 93.98) (width 1) (layer B.Cu) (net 15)))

